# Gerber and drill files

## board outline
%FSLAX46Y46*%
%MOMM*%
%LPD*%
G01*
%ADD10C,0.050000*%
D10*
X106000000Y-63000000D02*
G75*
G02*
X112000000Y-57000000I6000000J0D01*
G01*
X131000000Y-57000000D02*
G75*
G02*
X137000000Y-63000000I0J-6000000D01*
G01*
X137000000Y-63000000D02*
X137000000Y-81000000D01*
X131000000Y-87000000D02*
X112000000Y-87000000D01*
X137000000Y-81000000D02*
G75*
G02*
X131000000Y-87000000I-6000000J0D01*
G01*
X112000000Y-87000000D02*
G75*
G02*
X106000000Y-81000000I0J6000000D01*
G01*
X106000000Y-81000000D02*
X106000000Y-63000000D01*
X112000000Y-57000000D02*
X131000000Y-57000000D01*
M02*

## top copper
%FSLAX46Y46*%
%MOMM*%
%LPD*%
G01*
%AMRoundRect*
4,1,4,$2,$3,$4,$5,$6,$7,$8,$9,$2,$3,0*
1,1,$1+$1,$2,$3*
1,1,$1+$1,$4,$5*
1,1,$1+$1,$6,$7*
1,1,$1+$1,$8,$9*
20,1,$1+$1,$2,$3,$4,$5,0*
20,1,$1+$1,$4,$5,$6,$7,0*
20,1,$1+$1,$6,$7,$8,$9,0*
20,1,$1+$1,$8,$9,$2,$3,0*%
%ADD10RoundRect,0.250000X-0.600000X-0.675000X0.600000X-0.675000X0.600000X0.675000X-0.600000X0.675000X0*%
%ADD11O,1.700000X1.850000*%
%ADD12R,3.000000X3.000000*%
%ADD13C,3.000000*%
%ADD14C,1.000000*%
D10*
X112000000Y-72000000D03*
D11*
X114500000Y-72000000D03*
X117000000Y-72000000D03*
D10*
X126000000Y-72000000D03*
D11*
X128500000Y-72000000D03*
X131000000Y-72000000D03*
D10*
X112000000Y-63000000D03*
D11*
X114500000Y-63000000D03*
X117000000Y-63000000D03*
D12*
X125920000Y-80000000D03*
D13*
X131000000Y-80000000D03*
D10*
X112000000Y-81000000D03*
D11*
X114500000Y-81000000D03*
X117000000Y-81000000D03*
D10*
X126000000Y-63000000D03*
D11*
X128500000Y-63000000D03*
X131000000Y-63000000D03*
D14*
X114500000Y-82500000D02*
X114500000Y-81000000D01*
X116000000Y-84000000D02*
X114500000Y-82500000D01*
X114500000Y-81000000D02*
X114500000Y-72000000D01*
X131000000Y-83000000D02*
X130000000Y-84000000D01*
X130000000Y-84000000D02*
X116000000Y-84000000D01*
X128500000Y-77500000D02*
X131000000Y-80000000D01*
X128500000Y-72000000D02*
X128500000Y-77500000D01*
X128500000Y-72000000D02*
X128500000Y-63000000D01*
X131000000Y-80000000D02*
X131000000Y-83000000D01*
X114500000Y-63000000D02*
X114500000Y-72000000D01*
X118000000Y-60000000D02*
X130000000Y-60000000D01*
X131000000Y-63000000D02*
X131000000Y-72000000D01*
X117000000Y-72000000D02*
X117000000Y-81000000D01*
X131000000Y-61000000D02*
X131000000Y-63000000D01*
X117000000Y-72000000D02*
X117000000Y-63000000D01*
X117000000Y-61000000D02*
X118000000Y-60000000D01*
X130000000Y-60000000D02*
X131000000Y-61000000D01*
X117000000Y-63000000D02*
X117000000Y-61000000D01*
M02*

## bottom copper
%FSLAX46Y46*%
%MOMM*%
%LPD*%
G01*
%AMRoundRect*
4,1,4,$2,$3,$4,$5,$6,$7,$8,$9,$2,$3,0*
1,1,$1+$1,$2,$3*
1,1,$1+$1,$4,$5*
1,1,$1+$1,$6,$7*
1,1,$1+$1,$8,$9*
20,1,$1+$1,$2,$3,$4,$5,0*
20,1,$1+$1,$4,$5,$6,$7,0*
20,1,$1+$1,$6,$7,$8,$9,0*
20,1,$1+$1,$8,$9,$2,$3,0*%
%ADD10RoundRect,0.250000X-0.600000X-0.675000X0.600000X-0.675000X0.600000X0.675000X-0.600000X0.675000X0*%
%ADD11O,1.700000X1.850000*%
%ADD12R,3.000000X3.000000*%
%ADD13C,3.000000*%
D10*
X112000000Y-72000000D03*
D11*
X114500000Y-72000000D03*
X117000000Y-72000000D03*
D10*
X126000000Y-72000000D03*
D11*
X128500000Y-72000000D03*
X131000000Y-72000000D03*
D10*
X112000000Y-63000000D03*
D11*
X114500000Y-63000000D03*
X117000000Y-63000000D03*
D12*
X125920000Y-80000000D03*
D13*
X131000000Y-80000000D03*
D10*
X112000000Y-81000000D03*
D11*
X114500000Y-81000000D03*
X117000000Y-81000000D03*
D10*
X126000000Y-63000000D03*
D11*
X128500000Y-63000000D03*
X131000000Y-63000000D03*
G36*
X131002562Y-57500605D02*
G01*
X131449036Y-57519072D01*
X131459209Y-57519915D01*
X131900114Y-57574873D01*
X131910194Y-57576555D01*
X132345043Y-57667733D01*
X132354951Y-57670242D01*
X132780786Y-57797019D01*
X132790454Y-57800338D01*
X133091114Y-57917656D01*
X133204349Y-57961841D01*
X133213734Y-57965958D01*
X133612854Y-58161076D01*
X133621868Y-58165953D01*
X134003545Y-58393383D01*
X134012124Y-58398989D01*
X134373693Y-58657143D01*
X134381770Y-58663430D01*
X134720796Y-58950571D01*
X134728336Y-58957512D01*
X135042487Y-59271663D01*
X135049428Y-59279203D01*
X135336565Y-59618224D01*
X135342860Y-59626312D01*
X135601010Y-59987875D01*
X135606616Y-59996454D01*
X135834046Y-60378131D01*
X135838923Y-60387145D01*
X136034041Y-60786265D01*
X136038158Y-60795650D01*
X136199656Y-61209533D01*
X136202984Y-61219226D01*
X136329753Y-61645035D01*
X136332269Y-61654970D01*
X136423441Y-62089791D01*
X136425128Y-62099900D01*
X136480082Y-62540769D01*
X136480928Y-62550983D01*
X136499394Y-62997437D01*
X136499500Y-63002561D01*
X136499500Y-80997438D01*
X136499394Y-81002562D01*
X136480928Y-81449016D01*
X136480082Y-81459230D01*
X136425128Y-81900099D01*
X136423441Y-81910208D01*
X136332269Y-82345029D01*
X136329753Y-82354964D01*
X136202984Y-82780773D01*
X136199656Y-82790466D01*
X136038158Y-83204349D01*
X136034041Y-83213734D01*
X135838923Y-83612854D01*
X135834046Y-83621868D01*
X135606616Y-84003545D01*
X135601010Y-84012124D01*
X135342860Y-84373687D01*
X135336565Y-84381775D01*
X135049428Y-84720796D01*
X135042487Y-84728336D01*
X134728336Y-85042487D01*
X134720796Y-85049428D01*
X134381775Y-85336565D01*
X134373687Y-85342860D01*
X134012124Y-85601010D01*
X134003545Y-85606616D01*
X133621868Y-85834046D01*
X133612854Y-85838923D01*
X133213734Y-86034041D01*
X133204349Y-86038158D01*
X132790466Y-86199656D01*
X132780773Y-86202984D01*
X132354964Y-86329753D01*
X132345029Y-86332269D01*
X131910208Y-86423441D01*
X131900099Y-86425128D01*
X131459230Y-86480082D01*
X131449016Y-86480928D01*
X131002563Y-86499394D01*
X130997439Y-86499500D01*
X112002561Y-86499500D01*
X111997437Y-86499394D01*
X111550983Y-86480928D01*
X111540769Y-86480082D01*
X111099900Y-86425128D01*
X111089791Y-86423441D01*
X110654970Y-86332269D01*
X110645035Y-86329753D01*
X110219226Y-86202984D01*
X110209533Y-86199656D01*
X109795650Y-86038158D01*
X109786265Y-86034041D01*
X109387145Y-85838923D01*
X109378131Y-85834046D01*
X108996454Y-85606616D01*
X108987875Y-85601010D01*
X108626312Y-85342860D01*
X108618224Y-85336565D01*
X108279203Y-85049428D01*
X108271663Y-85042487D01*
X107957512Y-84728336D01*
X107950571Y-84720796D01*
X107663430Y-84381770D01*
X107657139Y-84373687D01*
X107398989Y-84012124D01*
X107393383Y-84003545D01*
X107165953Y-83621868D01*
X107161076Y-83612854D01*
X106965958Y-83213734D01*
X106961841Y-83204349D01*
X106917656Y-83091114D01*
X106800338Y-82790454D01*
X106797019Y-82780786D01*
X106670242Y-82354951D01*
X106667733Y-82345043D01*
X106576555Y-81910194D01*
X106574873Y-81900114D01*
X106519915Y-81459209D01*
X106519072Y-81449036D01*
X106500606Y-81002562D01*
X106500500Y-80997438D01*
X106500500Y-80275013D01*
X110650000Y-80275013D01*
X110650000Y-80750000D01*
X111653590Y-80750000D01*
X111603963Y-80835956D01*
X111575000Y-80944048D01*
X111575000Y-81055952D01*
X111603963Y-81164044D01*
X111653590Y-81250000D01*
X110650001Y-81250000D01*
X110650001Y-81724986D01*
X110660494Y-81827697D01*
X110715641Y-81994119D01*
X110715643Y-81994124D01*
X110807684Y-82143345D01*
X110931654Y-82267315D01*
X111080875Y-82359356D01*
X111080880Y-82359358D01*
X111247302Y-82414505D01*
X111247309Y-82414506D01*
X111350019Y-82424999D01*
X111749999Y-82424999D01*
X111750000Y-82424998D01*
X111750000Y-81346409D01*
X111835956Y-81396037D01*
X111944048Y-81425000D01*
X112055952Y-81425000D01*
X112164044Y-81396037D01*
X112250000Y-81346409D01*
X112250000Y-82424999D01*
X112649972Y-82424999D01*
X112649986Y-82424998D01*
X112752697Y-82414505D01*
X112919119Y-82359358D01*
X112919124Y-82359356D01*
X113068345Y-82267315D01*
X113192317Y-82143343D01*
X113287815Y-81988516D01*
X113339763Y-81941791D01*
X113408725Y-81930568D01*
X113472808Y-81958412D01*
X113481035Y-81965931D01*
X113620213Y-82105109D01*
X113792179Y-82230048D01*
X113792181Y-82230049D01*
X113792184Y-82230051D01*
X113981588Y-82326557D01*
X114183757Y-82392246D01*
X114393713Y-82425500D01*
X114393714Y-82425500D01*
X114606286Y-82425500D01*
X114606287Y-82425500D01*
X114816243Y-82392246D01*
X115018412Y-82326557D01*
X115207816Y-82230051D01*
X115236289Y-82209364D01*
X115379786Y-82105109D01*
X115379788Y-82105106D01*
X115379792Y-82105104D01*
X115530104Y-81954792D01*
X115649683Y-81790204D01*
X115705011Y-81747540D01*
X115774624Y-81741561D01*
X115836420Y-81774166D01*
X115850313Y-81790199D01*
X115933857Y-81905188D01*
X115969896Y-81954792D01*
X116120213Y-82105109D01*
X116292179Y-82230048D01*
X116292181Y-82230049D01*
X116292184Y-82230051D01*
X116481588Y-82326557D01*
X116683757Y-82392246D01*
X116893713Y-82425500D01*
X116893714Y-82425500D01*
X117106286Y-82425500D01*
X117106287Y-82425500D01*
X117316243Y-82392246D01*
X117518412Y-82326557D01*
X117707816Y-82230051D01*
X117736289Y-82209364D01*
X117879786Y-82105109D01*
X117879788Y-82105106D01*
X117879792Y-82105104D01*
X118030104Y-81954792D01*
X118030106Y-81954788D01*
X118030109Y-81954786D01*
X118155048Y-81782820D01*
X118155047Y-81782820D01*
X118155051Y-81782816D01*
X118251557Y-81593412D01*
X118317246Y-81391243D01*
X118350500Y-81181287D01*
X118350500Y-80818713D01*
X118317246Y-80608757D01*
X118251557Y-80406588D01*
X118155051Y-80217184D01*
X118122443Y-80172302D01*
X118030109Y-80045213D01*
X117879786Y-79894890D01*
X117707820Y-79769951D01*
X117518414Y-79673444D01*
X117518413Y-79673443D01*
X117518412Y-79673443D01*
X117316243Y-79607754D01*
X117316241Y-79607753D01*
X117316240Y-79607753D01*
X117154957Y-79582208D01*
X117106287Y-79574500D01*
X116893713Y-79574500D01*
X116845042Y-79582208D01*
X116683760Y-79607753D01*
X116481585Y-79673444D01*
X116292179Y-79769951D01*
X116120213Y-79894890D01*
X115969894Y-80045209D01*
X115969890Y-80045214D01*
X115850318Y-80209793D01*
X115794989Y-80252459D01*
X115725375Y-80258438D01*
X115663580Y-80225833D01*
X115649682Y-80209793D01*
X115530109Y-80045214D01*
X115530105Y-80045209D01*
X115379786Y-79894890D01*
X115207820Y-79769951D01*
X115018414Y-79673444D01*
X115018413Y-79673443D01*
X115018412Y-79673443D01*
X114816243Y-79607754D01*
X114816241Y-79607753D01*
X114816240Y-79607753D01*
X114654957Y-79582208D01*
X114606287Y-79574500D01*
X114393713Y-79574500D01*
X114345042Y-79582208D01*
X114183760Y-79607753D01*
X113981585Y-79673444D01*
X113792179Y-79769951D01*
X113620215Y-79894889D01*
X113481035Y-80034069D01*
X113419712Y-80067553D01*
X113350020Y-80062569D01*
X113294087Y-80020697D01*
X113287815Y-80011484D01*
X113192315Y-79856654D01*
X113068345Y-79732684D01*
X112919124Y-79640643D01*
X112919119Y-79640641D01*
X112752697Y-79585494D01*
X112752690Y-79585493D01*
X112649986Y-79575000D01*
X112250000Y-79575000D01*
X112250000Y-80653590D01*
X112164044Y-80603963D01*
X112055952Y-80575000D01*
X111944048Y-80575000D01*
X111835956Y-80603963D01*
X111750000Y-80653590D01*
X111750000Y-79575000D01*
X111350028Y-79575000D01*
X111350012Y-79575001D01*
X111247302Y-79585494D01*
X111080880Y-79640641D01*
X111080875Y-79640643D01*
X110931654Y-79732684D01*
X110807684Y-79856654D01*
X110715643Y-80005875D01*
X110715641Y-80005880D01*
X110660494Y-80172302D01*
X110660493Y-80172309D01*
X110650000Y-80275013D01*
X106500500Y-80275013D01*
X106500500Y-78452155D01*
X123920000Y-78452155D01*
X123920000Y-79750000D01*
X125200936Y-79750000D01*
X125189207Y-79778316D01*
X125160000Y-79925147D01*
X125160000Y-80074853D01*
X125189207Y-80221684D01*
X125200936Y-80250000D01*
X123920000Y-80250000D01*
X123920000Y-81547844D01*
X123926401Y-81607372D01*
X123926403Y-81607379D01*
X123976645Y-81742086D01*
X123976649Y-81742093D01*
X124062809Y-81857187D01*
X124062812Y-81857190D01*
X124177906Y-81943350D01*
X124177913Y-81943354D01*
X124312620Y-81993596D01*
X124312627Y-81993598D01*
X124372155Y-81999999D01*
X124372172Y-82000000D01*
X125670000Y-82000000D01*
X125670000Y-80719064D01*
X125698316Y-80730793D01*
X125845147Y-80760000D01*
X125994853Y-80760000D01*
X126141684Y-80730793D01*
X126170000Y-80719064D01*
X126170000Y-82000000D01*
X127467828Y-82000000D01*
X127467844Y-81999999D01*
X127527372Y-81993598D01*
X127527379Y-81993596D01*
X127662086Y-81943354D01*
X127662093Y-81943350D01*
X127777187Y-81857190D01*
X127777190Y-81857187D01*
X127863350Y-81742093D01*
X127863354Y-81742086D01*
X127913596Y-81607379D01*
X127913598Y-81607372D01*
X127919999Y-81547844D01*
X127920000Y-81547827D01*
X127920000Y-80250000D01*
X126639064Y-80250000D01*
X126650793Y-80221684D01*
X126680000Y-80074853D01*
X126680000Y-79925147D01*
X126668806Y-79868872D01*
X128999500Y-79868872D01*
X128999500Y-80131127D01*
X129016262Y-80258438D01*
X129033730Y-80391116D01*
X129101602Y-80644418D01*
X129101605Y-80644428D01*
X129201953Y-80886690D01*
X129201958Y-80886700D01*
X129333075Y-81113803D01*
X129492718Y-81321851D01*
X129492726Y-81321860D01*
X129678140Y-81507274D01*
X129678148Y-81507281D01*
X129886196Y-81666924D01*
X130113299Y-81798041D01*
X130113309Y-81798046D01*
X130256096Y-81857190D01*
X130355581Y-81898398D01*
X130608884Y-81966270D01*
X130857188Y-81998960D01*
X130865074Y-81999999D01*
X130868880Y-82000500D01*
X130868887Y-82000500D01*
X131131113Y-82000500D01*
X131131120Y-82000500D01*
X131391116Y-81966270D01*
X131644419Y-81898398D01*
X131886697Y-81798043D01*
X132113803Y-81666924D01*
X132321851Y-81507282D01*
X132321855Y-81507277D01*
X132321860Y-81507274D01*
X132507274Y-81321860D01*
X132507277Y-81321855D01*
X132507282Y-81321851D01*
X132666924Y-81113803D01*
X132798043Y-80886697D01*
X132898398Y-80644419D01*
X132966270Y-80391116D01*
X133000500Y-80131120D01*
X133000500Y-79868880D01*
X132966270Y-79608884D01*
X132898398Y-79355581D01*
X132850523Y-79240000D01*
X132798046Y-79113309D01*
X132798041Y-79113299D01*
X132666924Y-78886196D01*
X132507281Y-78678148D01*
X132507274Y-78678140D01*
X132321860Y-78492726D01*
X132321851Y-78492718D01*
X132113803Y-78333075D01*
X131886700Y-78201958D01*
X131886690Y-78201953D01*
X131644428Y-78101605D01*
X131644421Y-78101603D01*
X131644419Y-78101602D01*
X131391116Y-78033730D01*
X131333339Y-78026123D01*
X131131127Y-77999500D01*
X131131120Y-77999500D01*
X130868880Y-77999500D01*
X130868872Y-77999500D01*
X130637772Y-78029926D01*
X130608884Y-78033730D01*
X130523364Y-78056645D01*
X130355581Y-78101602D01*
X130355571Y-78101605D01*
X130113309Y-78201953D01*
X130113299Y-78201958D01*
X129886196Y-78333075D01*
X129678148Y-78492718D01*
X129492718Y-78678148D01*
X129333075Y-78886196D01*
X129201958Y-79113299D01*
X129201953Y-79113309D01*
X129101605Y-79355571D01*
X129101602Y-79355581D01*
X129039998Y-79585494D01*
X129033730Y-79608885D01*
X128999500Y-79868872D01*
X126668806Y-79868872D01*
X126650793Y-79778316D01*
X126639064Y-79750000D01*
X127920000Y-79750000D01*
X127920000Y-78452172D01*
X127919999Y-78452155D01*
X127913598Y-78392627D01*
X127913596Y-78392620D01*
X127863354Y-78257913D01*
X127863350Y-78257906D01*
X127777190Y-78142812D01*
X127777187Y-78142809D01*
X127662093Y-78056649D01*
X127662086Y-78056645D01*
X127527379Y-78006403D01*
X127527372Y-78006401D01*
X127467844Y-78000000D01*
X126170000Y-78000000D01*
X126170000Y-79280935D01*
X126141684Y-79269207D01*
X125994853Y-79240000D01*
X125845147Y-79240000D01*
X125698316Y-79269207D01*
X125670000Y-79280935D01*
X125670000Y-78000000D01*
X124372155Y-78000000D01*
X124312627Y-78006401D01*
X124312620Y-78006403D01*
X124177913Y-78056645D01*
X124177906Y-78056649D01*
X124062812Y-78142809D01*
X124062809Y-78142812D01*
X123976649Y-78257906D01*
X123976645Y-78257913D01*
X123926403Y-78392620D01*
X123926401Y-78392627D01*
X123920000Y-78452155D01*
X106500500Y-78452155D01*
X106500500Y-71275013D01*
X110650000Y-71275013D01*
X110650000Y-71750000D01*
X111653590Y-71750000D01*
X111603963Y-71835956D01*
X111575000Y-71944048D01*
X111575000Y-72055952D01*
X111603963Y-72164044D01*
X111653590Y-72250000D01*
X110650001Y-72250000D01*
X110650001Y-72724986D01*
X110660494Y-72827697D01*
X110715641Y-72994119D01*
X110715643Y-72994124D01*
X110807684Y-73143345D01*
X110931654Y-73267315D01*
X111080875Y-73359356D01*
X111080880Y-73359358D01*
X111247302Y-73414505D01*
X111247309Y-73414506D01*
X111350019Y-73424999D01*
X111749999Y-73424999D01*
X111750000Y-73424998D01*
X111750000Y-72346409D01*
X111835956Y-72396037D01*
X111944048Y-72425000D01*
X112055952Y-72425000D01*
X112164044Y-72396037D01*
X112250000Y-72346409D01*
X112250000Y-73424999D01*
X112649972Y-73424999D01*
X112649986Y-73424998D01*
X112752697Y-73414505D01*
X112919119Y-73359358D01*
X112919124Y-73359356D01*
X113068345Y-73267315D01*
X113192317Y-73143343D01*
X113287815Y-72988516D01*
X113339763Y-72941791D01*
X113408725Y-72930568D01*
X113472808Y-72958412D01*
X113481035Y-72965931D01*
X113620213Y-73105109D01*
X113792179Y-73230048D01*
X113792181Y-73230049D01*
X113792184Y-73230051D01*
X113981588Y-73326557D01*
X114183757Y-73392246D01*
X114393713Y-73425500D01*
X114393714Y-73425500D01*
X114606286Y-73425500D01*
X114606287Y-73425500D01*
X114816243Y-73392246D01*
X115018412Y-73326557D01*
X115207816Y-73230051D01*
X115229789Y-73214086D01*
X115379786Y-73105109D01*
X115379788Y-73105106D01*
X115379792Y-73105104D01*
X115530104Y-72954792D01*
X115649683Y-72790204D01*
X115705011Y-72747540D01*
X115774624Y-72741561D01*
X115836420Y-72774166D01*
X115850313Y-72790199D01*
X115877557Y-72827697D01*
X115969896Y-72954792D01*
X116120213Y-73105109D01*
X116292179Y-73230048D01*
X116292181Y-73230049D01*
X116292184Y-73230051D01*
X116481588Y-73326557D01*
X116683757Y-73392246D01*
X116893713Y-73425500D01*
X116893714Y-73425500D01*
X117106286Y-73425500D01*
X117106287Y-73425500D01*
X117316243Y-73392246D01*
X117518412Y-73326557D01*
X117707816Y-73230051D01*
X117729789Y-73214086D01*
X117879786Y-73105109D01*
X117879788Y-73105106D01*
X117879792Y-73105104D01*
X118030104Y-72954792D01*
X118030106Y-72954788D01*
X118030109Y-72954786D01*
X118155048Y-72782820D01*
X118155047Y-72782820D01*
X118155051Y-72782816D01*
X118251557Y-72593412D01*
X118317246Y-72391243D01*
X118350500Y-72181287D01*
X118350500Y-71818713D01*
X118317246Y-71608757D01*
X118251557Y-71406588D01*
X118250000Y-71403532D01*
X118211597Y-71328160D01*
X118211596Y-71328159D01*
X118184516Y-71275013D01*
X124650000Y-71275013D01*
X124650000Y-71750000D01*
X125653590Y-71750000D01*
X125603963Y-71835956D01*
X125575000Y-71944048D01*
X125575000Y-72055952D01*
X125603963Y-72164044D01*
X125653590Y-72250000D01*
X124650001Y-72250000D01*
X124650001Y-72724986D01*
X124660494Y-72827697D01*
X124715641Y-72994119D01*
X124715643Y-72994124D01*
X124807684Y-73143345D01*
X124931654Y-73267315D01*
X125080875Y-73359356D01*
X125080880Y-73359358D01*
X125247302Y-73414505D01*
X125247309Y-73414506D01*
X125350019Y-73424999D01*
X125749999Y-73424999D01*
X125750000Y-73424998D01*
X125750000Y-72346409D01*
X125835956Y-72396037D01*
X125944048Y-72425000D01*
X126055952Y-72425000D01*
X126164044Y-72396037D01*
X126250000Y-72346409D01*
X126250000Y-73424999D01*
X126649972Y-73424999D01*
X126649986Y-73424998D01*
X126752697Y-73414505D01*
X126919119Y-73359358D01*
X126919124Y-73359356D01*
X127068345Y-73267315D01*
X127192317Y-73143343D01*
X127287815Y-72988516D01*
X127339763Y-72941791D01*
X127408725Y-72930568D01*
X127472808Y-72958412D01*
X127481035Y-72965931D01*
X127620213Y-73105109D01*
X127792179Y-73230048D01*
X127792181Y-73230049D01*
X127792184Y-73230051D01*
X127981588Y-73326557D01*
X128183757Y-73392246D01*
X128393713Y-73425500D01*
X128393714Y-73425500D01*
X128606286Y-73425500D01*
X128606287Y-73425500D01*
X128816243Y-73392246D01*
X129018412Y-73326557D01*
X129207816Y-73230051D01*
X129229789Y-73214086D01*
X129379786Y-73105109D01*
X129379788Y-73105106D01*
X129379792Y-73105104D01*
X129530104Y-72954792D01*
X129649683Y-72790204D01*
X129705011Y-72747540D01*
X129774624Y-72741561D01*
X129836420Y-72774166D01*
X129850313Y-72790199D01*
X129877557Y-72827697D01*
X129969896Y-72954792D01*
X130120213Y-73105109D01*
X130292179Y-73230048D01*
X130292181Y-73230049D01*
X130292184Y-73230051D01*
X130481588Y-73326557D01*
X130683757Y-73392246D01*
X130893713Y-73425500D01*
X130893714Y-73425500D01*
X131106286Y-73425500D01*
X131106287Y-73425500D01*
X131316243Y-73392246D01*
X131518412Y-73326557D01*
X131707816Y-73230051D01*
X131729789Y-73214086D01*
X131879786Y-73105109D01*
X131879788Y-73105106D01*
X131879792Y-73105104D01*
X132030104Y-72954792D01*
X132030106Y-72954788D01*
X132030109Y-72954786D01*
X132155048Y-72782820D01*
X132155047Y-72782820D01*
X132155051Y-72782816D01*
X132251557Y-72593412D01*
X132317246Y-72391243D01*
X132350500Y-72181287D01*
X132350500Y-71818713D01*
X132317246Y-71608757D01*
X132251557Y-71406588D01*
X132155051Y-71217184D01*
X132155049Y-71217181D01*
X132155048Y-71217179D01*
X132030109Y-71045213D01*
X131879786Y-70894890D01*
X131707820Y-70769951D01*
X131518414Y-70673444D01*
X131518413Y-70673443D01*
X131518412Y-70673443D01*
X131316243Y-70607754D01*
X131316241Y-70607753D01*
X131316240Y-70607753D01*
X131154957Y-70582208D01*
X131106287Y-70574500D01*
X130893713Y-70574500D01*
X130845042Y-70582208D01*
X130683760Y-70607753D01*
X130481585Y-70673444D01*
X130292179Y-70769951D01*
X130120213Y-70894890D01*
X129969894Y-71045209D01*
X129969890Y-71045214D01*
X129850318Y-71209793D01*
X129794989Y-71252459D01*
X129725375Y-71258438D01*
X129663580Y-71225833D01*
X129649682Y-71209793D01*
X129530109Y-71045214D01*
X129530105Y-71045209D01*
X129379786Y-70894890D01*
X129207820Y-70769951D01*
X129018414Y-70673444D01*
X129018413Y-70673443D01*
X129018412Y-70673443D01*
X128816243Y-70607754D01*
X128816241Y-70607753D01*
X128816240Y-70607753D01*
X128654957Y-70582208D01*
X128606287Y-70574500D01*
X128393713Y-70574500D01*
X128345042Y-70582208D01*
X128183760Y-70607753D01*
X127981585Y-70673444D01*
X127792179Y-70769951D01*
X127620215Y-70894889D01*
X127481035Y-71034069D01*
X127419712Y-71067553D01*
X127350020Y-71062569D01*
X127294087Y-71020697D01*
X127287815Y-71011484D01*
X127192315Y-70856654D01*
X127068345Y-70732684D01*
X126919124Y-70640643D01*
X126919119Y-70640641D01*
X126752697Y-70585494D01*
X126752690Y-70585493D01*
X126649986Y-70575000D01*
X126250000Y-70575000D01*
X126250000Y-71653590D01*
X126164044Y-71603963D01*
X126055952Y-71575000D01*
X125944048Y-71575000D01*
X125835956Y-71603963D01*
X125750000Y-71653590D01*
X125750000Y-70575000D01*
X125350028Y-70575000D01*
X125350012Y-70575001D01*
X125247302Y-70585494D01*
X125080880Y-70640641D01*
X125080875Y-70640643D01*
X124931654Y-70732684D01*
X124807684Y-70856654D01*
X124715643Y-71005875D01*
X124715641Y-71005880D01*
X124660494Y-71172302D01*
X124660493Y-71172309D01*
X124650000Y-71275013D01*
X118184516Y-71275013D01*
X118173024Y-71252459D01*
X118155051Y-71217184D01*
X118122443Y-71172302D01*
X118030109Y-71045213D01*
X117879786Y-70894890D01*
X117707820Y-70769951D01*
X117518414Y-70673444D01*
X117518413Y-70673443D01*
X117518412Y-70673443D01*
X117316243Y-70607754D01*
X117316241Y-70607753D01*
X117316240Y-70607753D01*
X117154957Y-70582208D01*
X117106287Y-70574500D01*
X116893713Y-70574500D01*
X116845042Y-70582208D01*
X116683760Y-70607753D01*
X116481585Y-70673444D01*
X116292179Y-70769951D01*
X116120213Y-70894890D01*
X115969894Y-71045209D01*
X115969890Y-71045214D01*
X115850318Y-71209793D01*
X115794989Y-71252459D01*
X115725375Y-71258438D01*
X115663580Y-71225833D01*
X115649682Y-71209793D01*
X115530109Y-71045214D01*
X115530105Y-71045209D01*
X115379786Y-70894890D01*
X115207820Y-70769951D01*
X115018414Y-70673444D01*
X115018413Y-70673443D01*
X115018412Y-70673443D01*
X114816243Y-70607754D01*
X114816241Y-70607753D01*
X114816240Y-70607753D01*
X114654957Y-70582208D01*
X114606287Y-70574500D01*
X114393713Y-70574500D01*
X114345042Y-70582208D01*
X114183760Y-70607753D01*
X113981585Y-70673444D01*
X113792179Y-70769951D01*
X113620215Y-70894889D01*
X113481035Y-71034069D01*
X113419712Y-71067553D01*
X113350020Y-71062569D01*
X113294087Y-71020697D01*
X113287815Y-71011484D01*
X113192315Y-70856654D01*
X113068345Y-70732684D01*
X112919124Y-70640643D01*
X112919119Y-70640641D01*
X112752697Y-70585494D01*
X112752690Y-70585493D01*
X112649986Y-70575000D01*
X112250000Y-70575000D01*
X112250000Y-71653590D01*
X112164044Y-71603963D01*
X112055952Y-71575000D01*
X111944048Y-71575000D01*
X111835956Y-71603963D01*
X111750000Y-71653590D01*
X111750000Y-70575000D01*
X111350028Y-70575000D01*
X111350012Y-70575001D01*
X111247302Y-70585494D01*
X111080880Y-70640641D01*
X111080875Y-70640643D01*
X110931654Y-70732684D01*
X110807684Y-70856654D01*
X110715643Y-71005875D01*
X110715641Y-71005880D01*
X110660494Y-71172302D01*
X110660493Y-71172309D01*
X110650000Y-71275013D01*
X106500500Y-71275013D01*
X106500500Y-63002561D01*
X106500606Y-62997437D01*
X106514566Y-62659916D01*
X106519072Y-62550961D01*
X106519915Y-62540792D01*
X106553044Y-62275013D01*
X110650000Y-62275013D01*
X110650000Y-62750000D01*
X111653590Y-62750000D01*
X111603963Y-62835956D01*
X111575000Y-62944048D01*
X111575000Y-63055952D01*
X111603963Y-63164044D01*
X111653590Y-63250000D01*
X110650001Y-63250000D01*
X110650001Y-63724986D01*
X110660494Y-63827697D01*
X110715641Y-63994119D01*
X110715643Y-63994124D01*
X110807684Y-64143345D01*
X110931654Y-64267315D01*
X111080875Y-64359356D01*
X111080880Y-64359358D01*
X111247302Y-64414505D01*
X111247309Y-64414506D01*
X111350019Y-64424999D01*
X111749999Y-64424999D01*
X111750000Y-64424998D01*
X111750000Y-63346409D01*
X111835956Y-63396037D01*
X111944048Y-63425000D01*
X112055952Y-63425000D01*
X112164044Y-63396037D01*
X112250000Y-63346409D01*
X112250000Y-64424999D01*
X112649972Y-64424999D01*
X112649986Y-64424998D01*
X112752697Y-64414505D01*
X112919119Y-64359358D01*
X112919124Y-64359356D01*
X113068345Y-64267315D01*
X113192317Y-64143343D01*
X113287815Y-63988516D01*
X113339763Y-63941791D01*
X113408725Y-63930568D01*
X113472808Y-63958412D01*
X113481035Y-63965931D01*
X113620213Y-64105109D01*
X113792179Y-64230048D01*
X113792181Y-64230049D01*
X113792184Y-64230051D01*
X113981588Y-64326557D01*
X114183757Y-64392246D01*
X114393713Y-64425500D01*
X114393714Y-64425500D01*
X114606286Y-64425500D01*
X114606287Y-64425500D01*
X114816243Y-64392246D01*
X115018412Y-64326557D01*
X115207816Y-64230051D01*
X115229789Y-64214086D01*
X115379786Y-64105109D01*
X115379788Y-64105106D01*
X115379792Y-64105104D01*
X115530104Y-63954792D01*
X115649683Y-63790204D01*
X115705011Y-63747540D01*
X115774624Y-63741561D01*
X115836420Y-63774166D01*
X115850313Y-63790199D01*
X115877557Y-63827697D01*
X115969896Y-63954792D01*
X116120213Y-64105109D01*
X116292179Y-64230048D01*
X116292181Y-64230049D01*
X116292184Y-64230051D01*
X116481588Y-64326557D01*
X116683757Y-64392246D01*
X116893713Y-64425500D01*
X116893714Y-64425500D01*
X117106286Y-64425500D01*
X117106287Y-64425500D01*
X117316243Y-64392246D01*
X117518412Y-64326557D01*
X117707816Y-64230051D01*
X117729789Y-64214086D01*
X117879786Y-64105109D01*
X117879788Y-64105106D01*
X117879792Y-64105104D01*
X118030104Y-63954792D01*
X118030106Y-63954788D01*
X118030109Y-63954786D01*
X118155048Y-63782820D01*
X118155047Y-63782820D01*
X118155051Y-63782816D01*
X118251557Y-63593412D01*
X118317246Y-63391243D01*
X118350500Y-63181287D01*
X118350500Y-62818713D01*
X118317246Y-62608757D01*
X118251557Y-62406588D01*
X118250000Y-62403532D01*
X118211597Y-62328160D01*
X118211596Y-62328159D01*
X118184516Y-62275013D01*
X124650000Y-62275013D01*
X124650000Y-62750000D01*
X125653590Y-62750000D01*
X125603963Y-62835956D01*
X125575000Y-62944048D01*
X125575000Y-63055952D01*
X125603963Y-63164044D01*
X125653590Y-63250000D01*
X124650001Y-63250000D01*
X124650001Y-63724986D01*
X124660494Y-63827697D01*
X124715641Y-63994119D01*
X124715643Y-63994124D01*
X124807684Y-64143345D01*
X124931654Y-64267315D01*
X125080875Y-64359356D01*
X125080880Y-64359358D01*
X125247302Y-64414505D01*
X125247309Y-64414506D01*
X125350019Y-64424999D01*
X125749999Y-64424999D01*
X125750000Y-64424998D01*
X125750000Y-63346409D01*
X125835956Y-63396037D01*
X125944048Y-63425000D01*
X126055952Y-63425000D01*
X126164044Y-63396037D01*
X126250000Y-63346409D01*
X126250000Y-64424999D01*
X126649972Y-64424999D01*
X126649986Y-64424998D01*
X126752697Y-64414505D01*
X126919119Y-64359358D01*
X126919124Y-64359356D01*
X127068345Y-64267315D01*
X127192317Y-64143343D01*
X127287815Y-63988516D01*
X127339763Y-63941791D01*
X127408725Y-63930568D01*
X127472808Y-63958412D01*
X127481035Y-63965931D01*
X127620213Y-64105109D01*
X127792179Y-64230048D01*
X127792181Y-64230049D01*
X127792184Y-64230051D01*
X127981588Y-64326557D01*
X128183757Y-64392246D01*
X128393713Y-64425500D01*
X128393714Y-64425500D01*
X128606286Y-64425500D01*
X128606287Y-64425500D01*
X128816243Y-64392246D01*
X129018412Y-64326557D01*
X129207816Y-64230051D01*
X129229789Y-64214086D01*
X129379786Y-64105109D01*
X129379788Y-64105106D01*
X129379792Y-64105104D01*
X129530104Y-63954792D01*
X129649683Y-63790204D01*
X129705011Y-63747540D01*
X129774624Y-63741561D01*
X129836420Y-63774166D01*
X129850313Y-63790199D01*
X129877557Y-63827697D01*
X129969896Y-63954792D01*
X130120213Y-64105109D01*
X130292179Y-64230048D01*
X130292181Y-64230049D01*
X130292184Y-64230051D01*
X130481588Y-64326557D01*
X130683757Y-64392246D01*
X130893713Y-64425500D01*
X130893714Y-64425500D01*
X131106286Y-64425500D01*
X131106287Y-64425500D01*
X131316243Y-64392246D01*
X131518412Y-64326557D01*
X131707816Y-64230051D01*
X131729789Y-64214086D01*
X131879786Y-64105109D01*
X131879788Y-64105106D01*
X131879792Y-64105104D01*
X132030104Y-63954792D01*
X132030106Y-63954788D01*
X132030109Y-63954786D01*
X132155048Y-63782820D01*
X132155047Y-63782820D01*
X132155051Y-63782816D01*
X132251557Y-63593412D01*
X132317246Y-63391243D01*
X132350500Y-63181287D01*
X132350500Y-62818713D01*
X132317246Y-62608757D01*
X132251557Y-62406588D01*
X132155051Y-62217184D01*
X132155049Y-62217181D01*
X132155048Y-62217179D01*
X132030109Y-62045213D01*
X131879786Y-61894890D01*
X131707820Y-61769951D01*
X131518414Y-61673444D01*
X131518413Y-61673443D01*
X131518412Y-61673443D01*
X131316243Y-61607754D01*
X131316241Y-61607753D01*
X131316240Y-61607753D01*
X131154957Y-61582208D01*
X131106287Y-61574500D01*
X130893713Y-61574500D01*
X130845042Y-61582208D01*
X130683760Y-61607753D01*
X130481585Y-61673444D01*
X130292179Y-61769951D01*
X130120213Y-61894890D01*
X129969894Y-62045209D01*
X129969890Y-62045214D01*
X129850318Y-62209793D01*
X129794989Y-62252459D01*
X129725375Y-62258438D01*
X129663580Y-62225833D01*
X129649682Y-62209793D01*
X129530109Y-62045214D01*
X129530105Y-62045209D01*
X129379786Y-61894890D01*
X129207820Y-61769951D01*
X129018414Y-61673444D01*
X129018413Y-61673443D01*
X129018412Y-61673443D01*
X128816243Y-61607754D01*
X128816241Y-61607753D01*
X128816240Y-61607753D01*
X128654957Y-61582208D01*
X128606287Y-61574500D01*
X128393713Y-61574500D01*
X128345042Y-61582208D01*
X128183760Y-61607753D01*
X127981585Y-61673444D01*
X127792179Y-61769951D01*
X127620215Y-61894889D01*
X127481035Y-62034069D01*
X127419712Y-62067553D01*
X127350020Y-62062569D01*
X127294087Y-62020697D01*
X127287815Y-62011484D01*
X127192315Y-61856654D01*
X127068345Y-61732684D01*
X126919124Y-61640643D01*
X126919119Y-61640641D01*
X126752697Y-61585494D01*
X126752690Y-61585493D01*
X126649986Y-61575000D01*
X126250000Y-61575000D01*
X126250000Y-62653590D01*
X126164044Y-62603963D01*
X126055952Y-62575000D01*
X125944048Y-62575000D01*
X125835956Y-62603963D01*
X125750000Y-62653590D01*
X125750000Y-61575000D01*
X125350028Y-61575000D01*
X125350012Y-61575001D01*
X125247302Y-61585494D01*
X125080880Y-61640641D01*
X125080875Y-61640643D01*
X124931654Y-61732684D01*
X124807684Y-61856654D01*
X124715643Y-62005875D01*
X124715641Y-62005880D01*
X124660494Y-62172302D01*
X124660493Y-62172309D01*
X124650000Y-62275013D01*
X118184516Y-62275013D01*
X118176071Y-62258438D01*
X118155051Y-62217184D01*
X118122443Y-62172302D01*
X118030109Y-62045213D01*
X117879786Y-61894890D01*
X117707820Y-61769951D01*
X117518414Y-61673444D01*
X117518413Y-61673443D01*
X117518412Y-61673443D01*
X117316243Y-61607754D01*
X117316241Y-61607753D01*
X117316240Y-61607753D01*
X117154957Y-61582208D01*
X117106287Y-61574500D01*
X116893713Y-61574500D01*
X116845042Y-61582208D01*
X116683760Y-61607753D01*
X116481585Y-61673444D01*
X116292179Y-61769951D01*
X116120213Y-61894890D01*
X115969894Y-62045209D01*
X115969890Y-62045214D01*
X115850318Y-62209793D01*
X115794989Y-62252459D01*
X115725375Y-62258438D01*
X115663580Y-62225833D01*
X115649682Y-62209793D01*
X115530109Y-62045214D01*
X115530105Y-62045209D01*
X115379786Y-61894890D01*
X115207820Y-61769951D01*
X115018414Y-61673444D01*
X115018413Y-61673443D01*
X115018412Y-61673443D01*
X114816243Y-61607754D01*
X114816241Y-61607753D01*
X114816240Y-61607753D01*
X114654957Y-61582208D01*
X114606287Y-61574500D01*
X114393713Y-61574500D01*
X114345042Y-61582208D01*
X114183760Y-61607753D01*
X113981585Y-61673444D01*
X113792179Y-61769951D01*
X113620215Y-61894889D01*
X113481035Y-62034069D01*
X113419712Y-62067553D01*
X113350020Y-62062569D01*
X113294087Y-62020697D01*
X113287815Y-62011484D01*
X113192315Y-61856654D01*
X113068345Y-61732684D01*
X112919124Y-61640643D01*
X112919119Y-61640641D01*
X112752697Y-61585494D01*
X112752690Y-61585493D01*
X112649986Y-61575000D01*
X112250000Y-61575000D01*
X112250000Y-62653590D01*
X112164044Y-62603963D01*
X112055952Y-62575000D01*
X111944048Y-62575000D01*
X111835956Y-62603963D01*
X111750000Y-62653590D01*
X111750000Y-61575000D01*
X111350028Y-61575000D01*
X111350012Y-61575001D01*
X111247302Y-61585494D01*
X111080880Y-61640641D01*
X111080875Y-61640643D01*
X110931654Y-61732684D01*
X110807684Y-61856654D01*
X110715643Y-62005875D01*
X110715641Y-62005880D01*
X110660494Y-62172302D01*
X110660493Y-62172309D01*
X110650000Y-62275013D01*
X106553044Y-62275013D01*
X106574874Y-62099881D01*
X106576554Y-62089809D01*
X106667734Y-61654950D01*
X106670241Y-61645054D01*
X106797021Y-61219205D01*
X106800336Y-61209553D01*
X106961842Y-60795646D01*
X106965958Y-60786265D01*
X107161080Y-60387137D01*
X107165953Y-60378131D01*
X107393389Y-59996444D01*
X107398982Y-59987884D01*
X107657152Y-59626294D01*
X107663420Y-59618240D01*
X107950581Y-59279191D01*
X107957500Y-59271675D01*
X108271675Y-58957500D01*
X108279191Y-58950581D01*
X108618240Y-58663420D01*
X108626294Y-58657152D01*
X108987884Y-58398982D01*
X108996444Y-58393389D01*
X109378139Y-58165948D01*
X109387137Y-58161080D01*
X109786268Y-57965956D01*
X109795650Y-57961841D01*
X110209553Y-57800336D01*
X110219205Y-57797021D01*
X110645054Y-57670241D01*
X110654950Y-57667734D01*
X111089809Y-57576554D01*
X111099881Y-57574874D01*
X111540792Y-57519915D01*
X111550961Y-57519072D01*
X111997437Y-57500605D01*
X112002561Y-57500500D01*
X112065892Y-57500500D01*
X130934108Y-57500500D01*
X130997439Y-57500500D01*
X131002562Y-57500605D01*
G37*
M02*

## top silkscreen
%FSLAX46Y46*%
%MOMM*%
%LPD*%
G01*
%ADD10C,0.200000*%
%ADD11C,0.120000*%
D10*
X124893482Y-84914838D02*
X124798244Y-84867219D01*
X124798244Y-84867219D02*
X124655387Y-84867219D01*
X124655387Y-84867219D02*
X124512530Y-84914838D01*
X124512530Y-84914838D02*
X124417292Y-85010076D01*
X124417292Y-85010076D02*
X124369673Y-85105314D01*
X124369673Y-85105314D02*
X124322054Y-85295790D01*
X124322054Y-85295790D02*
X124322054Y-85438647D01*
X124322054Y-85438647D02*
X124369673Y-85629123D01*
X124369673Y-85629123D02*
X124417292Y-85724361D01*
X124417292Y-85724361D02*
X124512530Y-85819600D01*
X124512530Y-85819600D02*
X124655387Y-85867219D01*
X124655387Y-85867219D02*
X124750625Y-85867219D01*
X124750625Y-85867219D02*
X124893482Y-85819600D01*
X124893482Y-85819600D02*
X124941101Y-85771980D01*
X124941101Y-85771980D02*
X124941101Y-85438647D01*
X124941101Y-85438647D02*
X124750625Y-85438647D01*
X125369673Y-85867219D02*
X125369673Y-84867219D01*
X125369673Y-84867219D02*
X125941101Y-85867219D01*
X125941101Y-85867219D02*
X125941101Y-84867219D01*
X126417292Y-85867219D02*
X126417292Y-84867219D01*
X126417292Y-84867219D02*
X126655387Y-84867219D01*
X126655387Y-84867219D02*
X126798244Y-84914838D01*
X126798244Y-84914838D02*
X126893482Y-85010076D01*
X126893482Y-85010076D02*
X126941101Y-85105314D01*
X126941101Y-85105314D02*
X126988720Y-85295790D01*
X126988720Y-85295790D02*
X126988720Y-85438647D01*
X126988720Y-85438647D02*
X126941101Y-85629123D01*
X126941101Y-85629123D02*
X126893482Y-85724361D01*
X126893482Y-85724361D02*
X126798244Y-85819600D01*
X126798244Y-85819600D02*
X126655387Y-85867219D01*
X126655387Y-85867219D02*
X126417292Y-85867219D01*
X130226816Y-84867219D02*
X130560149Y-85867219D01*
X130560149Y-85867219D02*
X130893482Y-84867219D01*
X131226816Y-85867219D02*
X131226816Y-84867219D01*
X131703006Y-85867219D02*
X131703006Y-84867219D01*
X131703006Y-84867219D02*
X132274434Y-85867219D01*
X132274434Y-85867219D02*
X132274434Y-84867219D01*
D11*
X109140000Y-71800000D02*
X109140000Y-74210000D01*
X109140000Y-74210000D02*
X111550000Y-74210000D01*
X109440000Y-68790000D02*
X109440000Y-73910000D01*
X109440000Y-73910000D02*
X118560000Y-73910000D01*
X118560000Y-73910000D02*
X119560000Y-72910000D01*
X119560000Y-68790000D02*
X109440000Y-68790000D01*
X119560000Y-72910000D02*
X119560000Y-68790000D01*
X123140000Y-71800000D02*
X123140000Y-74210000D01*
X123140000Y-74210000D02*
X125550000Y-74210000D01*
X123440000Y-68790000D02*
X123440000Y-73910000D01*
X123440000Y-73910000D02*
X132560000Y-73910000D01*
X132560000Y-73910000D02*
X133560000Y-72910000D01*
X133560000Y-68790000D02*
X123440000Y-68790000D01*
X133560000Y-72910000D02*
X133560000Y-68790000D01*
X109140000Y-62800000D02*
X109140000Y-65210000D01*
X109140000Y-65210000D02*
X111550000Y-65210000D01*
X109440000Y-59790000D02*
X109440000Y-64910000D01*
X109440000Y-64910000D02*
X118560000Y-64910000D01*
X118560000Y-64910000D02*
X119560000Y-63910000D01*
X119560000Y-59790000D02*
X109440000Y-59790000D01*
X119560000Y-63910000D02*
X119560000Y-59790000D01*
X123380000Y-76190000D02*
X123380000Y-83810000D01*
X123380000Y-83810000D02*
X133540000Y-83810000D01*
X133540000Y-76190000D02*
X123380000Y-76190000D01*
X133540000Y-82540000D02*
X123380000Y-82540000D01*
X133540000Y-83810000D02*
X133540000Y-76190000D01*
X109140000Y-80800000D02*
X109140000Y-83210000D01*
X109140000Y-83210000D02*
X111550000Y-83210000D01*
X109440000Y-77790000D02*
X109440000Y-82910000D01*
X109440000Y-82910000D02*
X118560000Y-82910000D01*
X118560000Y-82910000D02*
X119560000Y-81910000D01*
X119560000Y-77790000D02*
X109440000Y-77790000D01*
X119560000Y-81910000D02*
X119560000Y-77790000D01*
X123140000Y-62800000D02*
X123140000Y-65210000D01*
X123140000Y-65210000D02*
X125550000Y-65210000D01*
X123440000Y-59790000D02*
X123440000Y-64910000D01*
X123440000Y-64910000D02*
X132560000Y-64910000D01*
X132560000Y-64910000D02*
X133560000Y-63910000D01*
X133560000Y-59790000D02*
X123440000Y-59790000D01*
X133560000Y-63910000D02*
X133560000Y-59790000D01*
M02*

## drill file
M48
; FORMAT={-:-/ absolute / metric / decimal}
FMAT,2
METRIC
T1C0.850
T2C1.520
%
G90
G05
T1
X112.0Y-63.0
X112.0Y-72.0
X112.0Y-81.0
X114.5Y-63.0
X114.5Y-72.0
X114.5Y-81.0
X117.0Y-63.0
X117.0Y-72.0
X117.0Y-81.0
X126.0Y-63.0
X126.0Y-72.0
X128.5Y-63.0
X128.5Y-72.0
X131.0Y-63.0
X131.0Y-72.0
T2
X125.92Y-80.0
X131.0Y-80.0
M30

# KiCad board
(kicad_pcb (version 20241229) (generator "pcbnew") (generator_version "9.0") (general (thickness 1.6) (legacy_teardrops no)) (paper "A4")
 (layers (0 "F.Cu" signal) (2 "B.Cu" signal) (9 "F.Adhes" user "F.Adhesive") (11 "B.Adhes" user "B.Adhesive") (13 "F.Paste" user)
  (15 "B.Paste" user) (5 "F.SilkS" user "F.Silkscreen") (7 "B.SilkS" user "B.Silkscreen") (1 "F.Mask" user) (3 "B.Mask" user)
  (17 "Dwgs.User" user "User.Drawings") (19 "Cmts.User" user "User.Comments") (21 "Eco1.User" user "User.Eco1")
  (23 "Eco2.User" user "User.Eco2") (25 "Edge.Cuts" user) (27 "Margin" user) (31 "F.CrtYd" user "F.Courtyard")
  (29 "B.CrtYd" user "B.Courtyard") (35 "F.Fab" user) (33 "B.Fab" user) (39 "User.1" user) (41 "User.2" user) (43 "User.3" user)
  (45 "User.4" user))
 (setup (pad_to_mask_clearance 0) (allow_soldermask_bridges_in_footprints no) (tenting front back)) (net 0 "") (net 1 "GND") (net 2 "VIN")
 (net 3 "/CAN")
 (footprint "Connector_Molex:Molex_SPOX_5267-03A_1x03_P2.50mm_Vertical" (layer "F.Cu") (at 112 72)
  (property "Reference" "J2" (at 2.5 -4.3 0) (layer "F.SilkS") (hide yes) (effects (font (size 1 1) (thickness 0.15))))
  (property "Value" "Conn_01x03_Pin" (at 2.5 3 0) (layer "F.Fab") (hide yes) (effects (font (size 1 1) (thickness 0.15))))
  (fp_line (start -2.86 -0.2) (end -2.86 2.21) (stroke (width 0.12) (type solid)) (layer "F.SilkS"))
  (fp_line (start -2.86 2.21) (end -0.45 2.21) (stroke (width 0.12) (type solid)) (layer "F.SilkS"))
  (fp_line (start -2.56 -3.21) (end -2.56 1.91) (stroke (width 0.12) (type solid)) (layer "F.SilkS"))
  (fp_line (start -2.56 1.91) (end 6.56 1.91) (stroke (width 0.12) (type solid)) (layer "F.SilkS"))
  (fp_line (start 6.56 1.91) (end 7.56 0.91) (stroke (width 0.12) (type solid)) (layer "F.SilkS"))
  (fp_line (start 7.56 -3.21) (end -2.56 -3.21) (stroke (width 0.12) (type solid)) (layer "F.SilkS"))
  (fp_line (start 7.56 0.91) (end 7.56 -3.21) (stroke (width 0.12) (type solid)) (layer "F.SilkS"))
  (pad "1" thru_hole roundrect (at 0 0) (size 1.7 1.85) (drill 0.85) (layers "*.Cu" "*.Mask") (remove_unused_layers no)
   (roundrect_rratio 0.147059) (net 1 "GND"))
  (pad "2" thru_hole oval (at 2.5 0) (size 1.7 1.85) (drill 0.85) (layers "*.Cu" "*.Mask") (remove_unused_layers no) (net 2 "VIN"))
  (pad "3" thru_hole oval (at 5 0) (size 1.7 1.85) (drill 0.85) (layers "*.Cu" "*.Mask") (remove_unused_layers no) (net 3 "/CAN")))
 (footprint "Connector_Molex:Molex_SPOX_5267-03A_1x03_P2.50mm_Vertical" (layer "F.Cu") (at 126 72)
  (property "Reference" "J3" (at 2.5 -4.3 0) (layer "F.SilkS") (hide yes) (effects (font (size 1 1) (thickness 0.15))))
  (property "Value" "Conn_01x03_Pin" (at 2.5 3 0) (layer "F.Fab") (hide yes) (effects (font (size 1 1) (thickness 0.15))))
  (fp_line (start -2.86 -0.2) (end -2.86 2.21) (stroke (width 0.12) (type solid)) (layer "F.SilkS"))
  (fp_line (start -2.86 2.21) (end -0.45 2.21) (stroke (width 0.12) (type solid)) (layer "F.SilkS"))
  (fp_line (start -2.56 -3.21) (end -2.56 1.91) (stroke (width 0.12) (type solid)) (layer "F.SilkS"))
  (fp_line (start -2.56 1.91) (end 6.56 1.91) (stroke (width 0.12) (type solid)) (layer "F.SilkS"))
  (fp_line (start 6.56 1.91) (end 7.56 0.91) (stroke (width 0.12) (type solid)) (layer "F.SilkS"))
  (fp_line (start 7.56 -3.21) (end -2.56 -3.21) (stroke (width 0.12) (type solid)) (layer "F.SilkS"))
  (fp_line (start 7.56 0.91) (end 7.56 -3.21) (stroke (width 0.12) (type solid)) (layer "F.SilkS"))
  (pad "1" thru_hole roundrect (at 0 0) (size 1.7 1.85) (drill 0.85) (layers "*.Cu" "*.Mask") (remove_unused_layers no)
   (roundrect_rratio 0.147059) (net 1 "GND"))
  (pad "2" thru_hole oval (at 2.5 0) (size 1.7 1.85) (drill 0.85) (layers "*.Cu" "*.Mask") (remove_unused_layers no) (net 2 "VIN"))
  (pad "3" thru_hole oval (at 5 0) (size 1.7 1.85) (drill 0.85) (layers "*.Cu" "*.Mask") (remove_unused_layers no) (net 3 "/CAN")))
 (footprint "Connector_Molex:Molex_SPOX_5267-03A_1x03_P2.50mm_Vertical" (layer "F.Cu") (at 112 63)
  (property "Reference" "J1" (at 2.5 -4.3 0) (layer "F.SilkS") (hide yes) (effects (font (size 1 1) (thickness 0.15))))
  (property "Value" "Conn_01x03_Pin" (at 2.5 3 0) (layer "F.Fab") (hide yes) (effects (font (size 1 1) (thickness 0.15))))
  (fp_line (start -2.86 -0.2) (end -2.86 2.21) (stroke (width 0.12) (type solid)) (layer "F.SilkS"))
  (fp_line (start -2.86 2.21) (end -0.45 2.21) (stroke (width 0.12) (type solid)) (layer "F.SilkS"))
  (fp_line (start -2.56 -3.21) (end -2.56 1.91) (stroke (width 0.12) (type solid)) (layer "F.SilkS"))
  (fp_line (start -2.56 1.91) (end 6.56 1.91) (stroke (width 0.12) (type solid)) (layer "F.SilkS"))
  (fp_line (start 6.56 1.91) (end 7.56 0.91) (stroke (width 0.12) (type solid)) (layer "F.SilkS"))
  (fp_line (start 7.56 -3.21) (end -2.56 -3.21) (stroke (width 0.12) (type solid)) (layer "F.SilkS"))
  (fp_line (start 7.56 0.91) (end 7.56 -3.21) (stroke (width 0.12) (type solid)) (layer "F.SilkS"))
  (pad "1" thru_hole roundrect (at 0 0) (size 1.7 1.85) (drill 0.85) (layers "*.Cu" "*.Mask") (remove_unused_layers no)
   (roundrect_rratio 0.147059) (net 1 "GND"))
  (pad "2" thru_hole oval (at 2.5 0) (size 1.7 1.85) (drill 0.85) (layers "*.Cu" "*.Mask") (remove_unused_layers no) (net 2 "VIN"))
  (pad "3" thru_hole oval (at 5 0) (size 1.7 1.85) (drill 0.85) (layers "*.Cu" "*.Mask") (remove_unused_layers no) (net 3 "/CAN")))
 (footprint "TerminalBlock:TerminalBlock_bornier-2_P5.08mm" (layer "F.Cu") (at 125.92 80)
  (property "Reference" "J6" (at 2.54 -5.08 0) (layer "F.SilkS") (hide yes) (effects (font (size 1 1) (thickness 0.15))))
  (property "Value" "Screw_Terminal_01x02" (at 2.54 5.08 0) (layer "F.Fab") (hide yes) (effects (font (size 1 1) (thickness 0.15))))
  (fp_line (start -2.54 -3.81) (end -2.54 3.81) (stroke (width 0.12) (type solid)) (layer "F.SilkS"))
  (fp_line (start -2.54 3.81) (end 7.62 3.81) (stroke (width 0.12) (type solid)) (layer "F.SilkS"))
  (fp_line (start 7.62 -3.81) (end -2.54 -3.81) (stroke (width 0.12) (type solid)) (layer "F.SilkS"))
  (fp_line (start 7.62 2.54) (end -2.54 2.54) (stroke (width 0.12) (type solid)) (layer "F.SilkS"))
  (fp_line (start 7.62 3.81) (end 7.62 -3.81) (stroke (width 0.12) (type solid)) (layer "F.SilkS"))
  (pad "1" thru_hole rect (at 0 0) (size 3 3) (drill 1.52) (layers "*.Cu" "*.Mask") (remove_unused_layers no) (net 1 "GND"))
  (pad "2" thru_hole circle (at 5.08 0) (size 3 3) (drill 1.52) (layers "*.Cu" "*.Mask") (remove_unused_layers no) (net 2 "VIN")))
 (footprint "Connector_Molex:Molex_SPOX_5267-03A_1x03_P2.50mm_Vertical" (layer "F.Cu") (at 112 81)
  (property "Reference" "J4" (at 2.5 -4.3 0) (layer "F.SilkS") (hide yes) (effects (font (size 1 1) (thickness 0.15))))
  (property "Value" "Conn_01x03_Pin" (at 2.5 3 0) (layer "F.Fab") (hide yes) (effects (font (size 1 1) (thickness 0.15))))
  (fp_line (start -2.86 -0.2) (end -2.86 2.21) (stroke (width 0.12) (type solid)) (layer "F.SilkS"))
  (fp_line (start -2.86 2.21) (end -0.45 2.21) (stroke (width 0.12) (type solid)) (layer "F.SilkS"))
  (fp_line (start -2.56 -3.21) (end -2.56 1.91) (stroke (width 0.12) (type solid)) (layer "F.SilkS"))
  (fp_line (start -2.56 1.91) (end 6.56 1.91) (stroke (width 0.12) (type solid)) (layer "F.SilkS"))
  (fp_line (start 6.56 1.91) (end 7.56 0.91) (stroke (width 0.12) (type solid)) (layer "F.SilkS"))
  (fp_line (start 7.56 -3.21) (end -2.56 -3.21) (stroke (width 0.12) (type solid)) (layer "F.SilkS"))
  (fp_line (start 7.56 0.91) (end 7.56 -3.21) (stroke (width 0.12) (type solid)) (layer "F.SilkS"))
  (pad "1" thru_hole roundrect (at 0 0) (size 1.7 1.85) (drill 0.85) (layers "*.Cu" "*.Mask") (remove_unused_layers no)
   (roundrect_rratio 0.147059) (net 1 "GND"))
  (pad "2" thru_hole oval (at 2.5 0) (size 1.7 1.85) (drill 0.85) (layers "*.Cu" "*.Mask") (remove_unused_layers no) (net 2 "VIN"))
  (pad "3" thru_hole oval (at 5 0) (size 1.7 1.85) (drill 0.85) (layers "*.Cu" "*.Mask") (remove_unused_layers no) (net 3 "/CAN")))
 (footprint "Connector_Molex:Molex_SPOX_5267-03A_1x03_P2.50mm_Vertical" (layer "F.Cu") (at 126 63)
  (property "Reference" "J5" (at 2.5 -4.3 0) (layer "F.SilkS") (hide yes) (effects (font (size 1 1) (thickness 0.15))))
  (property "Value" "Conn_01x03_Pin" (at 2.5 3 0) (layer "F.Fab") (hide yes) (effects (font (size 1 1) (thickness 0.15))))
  (fp_line (start -2.86 -0.2) (end -2.86 2.21) (stroke (width 0.12) (type solid)) (layer "F.SilkS"))
  (fp_line (start -2.86 2.21) (end -0.45 2.21) (stroke (width 0.12) (type solid)) (layer "F.SilkS"))
  (fp_line (start -2.56 -3.21) (end -2.56 1.91) (stroke (width 0.12) (type solid)) (layer "F.SilkS"))
  (fp_line (start -2.56 1.91) (end 6.56 1.91) (stroke (width 0.12) (type solid)) (layer "F.SilkS"))
  (fp_line (start 6.56 1.91) (end 7.56 0.91) (stroke (width 0.12) (type solid)) (layer "F.SilkS"))
  (fp_line (start 7.56 -3.21) (end -2.56 -3.21) (stroke (width 0.12) (type solid)) (layer "F.SilkS"))
  (fp_line (start 7.56 0.91) (end 7.56 -3.21) (stroke (width 0.12) (type solid)) (layer "F.SilkS"))
  (pad "1" thru_hole roundrect (at 0 0) (size 1.7 1.85) (drill 0.85) (layers "*.Cu" "*.Mask") (remove_unused_layers no)
   (roundrect_rratio 0.147059) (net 1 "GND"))
  (pad "2" thru_hole oval (at 2.5 0) (size 1.7 1.85) (drill 0.85) (layers "*.Cu" "*.Mask") (remove_unused_layers no) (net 2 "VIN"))
  (pad "3" thru_hole oval (at 5 0) (size 1.7 1.85) (drill 0.85) (layers "*.Cu" "*.Mask") (remove_unused_layers no) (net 3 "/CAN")))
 (gr_arc (start 106 63) (mid 107.757359 58.757359) (end 112 57) (stroke (width 0.05) (type default)) (layer "Edge.Cuts"))
 (gr_arc (start 131 57) (mid 135.242641 58.757359) (end 137 63) (stroke (width 0.05) (type default)) (layer "Edge.Cuts"))
 (gr_line (start 137 63) (end 137 81) (stroke (width 0.05) (type default)) (layer "Edge.Cuts"))
 (gr_line (start 131 87) (end 112 87) (stroke (width 0.05) (type default)) (layer "Edge.Cuts"))
 (gr_arc (start 137 81) (mid 135.242641 85.242641) (end 131 87) (stroke (width 0.05) (type default)) (layer "Edge.Cuts"))
 (gr_arc (start 112 87) (mid 107.757359 85.242641) (end 106 81) (stroke (width 0.05) (type default)) (layer "Edge.Cuts"))
 (gr_line (start 106 81) (end 106 63) (stroke (width 0.05) (type default)) (layer "Edge.Cuts"))
 (gr_line (start 112 57) (end 131 57) (stroke (width 0.05) (type default)) (layer "Edge.Cuts"))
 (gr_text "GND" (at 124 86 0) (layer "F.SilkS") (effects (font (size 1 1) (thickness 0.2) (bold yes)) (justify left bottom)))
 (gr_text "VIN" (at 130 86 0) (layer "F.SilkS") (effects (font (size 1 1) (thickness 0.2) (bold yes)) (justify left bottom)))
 (segment (start 114.5 82.5) (end 114.5 81) (width 1) (layer "F.Cu") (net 2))
 (segment (start 116 84) (end 114.5 82.5) (width 1) (layer "F.Cu") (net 2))
 (segment (start 114.5 81) (end 114.5 72) (width 1) (layer "F.Cu") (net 2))
 (segment (start 131 83) (end 130 84) (width 1) (layer "F.Cu") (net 2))
 (segment (start 130 84) (end 116 84) (width 1) (layer "F.Cu") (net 2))
 (segment (start 128.5 77.5) (end 131 80) (width 1) (layer "F.Cu") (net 2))
 (segment (start 128.5 72) (end 128.5 77.5) (width 1) (layer "F.Cu") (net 2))
 (segment (start 128.5 72) (end 128.5 63) (width 1) (layer "F.Cu") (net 2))
 (segment (start 131 80) (end 131 83) (width 1) (layer "F.Cu") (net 2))
 (segment (start 114.5 63) (end 114.5 72) (width 1) (layer "F.Cu") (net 2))
 (segment (start 118 60) (end 130 60) (width 1) (layer "F.Cu") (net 3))
 (segment (start 131 63) (end 131 72) (width 1) (layer "F.Cu") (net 3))
 (segment (start 117 72) (end 117 81) (width 1) (layer "F.Cu") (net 3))
 (segment (start 131 61) (end 131 63) (width 1) (layer "F.Cu") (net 3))
 (segment (start 117 72) (end 117 63) (width 1) (layer "F.Cu") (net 3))
 (segment (start 117 61) (end 118 60) (width 1) (layer "F.Cu") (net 3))
 (segment (start 130 60) (end 131 61) (width 1) (layer "F.Cu") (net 3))
 (segment (start 117 63) (end 117 61) (width 1) (layer "F.Cu") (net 3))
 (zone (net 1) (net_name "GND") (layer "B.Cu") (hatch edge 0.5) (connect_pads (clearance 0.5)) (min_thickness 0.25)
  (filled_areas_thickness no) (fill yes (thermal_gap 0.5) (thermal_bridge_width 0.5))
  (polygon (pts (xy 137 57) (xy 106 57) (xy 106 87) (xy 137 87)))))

